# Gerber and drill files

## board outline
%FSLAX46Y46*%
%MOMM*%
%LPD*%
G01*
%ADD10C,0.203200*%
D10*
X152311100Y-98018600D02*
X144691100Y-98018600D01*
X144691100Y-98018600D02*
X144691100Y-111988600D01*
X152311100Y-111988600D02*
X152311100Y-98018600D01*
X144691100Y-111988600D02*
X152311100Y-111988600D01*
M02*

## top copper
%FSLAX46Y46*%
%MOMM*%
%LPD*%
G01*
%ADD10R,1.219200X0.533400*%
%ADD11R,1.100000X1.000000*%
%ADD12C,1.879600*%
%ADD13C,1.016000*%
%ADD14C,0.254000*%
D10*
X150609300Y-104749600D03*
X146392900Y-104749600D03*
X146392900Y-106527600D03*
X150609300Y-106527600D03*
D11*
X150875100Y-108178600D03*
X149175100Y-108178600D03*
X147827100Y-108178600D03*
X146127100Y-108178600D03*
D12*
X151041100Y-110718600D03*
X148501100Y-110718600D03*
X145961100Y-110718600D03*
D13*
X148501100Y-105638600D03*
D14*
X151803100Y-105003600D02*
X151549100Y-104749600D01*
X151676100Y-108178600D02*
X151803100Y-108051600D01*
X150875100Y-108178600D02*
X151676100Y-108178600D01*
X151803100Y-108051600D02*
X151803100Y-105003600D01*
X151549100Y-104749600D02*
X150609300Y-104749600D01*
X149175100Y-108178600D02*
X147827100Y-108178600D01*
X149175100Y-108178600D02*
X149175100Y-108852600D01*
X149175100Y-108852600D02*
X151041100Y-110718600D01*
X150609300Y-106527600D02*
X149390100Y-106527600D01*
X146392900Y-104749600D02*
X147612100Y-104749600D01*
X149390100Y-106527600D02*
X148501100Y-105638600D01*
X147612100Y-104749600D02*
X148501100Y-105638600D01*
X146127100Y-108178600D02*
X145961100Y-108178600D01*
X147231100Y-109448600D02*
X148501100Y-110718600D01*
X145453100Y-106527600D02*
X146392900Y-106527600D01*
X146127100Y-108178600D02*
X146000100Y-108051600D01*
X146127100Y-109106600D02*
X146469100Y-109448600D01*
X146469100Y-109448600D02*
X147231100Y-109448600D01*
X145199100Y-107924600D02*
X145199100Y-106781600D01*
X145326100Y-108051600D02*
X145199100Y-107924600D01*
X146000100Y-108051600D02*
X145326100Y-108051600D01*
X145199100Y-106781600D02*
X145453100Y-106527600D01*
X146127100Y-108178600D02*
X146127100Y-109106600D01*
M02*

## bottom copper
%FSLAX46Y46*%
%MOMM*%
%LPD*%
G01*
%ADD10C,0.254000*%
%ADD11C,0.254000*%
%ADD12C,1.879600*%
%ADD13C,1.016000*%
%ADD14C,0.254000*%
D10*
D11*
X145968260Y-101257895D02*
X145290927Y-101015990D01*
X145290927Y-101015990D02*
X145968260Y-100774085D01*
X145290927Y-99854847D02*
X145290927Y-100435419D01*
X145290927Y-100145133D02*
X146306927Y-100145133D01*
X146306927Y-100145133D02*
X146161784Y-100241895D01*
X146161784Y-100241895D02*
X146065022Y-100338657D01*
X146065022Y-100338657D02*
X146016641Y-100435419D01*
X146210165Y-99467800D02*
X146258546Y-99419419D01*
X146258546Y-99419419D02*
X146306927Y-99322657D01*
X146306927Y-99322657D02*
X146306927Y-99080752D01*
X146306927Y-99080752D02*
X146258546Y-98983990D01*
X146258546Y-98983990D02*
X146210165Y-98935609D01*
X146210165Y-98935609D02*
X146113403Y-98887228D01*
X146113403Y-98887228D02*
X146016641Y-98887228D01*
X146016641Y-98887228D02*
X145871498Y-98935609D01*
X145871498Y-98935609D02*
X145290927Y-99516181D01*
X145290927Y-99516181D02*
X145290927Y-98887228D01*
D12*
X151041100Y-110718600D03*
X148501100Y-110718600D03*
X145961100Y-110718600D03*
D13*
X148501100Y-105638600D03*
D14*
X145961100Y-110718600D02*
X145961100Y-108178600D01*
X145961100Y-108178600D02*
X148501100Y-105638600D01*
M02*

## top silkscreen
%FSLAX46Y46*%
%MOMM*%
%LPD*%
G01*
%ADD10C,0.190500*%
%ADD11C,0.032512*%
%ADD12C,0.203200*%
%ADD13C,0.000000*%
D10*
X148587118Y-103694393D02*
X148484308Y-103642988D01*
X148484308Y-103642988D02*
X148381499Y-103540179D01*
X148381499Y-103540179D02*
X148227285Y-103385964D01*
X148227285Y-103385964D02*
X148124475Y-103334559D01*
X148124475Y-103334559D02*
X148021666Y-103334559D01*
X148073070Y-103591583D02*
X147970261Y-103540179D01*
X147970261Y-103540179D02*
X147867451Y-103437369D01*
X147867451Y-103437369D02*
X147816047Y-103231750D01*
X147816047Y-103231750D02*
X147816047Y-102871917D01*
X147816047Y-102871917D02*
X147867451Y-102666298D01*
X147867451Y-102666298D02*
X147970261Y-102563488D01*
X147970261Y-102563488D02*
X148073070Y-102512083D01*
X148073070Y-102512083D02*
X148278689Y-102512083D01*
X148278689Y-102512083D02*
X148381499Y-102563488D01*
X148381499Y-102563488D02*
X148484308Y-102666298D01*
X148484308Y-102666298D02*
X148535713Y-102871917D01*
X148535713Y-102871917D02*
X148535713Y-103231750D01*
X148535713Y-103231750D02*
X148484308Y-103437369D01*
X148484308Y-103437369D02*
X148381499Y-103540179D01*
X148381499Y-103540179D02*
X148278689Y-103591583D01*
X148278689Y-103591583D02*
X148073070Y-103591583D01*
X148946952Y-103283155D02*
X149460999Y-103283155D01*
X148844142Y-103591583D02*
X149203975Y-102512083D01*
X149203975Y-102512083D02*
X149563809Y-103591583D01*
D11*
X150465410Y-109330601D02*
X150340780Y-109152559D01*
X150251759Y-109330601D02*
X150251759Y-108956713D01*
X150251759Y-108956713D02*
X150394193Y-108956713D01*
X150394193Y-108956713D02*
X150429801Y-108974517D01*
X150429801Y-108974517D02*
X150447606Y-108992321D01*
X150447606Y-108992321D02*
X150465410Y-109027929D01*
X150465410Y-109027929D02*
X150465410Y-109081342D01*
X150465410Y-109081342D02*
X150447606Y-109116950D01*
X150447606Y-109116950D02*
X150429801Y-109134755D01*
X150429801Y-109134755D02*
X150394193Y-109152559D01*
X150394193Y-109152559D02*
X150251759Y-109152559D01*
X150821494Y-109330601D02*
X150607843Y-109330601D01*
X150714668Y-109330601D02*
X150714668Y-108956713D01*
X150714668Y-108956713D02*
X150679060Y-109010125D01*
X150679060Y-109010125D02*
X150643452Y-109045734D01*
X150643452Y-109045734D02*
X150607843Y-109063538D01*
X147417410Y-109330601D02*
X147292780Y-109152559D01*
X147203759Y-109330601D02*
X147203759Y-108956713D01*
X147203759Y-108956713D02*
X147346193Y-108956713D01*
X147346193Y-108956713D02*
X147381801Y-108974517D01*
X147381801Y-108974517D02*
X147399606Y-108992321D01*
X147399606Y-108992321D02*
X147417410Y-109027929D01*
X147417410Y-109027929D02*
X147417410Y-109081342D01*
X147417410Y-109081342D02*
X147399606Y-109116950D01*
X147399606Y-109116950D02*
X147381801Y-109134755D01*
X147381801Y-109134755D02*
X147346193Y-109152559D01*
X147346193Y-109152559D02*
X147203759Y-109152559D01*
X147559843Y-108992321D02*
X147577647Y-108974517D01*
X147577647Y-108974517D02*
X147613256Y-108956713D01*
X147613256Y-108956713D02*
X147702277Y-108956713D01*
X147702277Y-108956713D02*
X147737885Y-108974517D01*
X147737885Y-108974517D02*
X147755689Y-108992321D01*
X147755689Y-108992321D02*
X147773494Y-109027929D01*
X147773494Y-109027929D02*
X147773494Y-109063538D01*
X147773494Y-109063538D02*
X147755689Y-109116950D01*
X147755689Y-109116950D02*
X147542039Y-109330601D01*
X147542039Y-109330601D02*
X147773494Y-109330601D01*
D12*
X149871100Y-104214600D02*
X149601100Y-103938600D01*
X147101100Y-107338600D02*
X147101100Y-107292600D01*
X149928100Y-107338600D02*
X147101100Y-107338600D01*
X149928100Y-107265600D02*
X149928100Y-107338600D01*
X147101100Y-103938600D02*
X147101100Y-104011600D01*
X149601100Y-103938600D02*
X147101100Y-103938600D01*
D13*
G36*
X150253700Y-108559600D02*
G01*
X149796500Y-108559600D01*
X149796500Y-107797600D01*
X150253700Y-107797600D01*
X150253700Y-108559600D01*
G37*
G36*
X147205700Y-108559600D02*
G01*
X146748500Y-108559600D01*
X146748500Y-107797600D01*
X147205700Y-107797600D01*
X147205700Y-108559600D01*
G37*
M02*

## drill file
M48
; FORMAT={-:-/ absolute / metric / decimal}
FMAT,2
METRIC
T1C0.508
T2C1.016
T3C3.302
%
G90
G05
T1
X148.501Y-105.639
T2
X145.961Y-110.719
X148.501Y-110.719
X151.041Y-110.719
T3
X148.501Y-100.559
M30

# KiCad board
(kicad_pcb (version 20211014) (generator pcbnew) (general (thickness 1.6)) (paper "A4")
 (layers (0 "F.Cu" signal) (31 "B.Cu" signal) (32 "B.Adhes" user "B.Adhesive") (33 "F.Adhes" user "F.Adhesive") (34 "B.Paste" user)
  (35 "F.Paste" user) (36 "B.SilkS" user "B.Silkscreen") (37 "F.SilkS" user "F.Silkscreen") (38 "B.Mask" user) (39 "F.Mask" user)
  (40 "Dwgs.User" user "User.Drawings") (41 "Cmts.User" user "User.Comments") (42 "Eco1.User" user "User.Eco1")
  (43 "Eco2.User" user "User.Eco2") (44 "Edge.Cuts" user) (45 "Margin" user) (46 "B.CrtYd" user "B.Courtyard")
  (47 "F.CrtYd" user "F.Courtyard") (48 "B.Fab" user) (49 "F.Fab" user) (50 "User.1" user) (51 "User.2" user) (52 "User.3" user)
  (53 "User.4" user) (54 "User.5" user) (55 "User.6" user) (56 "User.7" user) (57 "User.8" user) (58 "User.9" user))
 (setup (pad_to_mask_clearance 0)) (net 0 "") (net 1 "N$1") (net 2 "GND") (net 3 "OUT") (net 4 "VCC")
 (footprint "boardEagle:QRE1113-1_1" (layer "F.Cu") (at 148.5011 105.6386 180)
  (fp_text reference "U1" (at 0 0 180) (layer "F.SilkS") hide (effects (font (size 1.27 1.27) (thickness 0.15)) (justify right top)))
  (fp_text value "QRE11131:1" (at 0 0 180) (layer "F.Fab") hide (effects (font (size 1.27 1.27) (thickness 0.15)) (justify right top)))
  (fp_line (start -1.37 1.424) (end -1.1 1.7) (layer "F.SilkS") (width 0.2032))
  (fp_line (start 1.4 -1.7) (end 1.4 -1.654) (layer "F.SilkS") (width 0.2032))
  (fp_line (start -1.427 -1.7) (end 1.4 -1.7) (layer "F.SilkS") (width 0.2032))
  (fp_line (start -1.427 -1.627) (end -1.427 -1.7) (layer "F.SilkS") (width 0.2032))
  (fp_line (start 1.4 1.7) (end 1.4 1.627) (layer "F.SilkS") (width 0.2032))
  (fp_line (start -1.1 1.7) (end 1.4 1.7) (layer "F.SilkS") (width 0.2032))
  (pad "1" smd rect (at -2.1082 0.889 180) (size 1.2192 0.5334) (layers "F.Cu" "F.Paste" "F.Mask") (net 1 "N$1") (solder_mask_margin 0.1016))
  (pad "2" smd rect (at 2.1082 0.889 180) (size 1.2192 0.5334) (layers "F.Cu" "F.Paste" "F.Mask") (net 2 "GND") (solder_mask_margin 0.1016))
  (pad "3" smd rect (at 2.1082 -0.889 180) (size 1.2192 0.5334) (layers "F.Cu" "F.Paste" "F.Mask") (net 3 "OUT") (solder_mask_margin 0.1016))
  (pad "4" smd rect (at -2.1082 -0.889 180) (size 1.2192 0.5334) (layers "F.Cu" "F.Paste" "F.Mask") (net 2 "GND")
   (solder_mask_margin 0.1016)))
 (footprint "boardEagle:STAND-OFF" (layer "F.Cu") (at 148.5011 100.5586)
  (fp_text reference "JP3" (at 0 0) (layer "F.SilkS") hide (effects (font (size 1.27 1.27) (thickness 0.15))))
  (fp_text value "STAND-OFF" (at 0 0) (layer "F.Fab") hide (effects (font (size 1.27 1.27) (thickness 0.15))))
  (pad "" np_thru_hole circle (at 0 0) (size 3.302 3.302) (drill 3.302) (layers *.Cu *.Mask)))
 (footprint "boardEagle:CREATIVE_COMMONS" (layer "F.Cu") (at 166.2811 119.6086)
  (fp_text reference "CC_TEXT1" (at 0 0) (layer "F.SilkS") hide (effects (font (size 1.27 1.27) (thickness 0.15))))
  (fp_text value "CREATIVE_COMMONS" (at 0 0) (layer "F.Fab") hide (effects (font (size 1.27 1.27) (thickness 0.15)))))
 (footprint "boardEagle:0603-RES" (layer "F.Cu") (at 150.0251 108.1786 180)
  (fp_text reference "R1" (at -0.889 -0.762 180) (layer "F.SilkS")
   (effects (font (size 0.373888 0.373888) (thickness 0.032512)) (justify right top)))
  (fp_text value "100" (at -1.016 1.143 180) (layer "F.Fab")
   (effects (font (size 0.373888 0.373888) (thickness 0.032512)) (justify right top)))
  (fp_poly (pts (xy -0.2286 0.381) (xy 0.2286 0.381) (xy 0.2286 -0.381) (xy -0.2286 -0.381)) (layer "F.SilkS") (width 0) (fill solid))
  (pad "1" smd rect (at -0.85 0 180) (size 1.1 1) (layers "F.Cu" "F.Paste" "F.Mask") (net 1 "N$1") (solder_mask_margin 0.1016))
  (pad "2" smd rect (at 0.85 0 180) (size 1.1 1) (layers "F.Cu" "F.Paste" "F.Mask") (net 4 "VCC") (solder_mask_margin 0.1016)))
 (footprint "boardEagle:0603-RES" (layer "F.Cu") (at 146.9771 108.1786 180)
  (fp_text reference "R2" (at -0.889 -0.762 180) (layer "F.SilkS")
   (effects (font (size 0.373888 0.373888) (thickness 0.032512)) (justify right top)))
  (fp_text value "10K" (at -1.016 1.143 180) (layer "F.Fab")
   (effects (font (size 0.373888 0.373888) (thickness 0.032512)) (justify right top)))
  (fp_poly (pts (xy -0.2286 0.381) (xy 0.2286 0.381) (xy 0.2286 -0.381) (xy -0.2286 -0.381)) (layer "F.SilkS") (width 0) (fill solid))
  (pad "1" smd rect (at -0.85 0 180) (size 1.1 1) (layers "F.Cu" "F.Paste" "F.Mask") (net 4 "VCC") (solder_mask_margin 0.1016))
  (pad "2" smd rect (at 0.85 0 180) (size 1.1 1) (layers "F.Cu" "F.Paste" "F.Mask") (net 3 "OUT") (solder_mask_margin 0.1016)))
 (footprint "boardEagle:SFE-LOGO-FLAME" (layer "B.Cu") (at 151.1681 105.1306 180)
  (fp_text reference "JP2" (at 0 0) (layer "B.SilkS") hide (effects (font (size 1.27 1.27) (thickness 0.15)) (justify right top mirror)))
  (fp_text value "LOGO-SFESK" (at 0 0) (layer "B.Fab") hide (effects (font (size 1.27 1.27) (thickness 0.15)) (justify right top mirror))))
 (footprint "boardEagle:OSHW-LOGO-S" (layer "B.Cu") (at 146.7231 103.8606 180)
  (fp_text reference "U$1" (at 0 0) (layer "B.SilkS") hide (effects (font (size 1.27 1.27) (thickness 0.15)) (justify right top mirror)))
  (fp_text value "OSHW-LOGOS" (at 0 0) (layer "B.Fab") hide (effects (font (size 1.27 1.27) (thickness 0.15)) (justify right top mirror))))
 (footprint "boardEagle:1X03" (layer "B.Cu") (at 151.0411 110.7186 180)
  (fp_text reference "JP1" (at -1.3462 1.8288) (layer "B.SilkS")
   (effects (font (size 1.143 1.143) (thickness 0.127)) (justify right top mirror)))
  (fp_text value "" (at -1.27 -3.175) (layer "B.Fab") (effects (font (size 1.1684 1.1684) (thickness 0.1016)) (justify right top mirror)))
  (pad "1" thru_hole circle (at 0 0 90) (size 1.8796 1.8796) (drill 1.016) (layers *.Cu *.Mask) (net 4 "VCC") (solder_mask_margin 0.1016))
  (pad "2" thru_hole circle (at 2.54 0 90) (size 1.8796 1.8796) (drill 1.016) (layers *.Cu *.Mask) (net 3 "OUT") (solder_mask_margin 0.1016))
  (pad "3" thru_hole circle (at 5.08 0 90) (size 1.8796 1.8796) (drill 1.016) (layers *.Cu *.Mask) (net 2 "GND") (solder_mask_margin 0.1016)))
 (gr_line (start 152.3111 98.0186) (end 144.6911 98.0186) (layer "Edge.Cuts") (width 0.2032))
 (gr_line (start 144.6911 98.0186) (end 144.6911 111.9886) (layer "Edge.Cuts") (width 0.2032))
 (gr_line (start 152.3111 111.9886) (end 152.3111 98.0186) (layer "Edge.Cuts") (width 0.2032))
 (gr_line (start 144.6911 111.9886) (end 152.3111 111.9886) (layer "Edge.Cuts") (width 0.2032))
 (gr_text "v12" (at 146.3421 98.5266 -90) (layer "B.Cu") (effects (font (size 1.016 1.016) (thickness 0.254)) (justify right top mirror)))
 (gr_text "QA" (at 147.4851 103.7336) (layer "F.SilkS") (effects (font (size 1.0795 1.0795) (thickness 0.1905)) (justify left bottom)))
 (segment (start 151.8031 105.0036) (end 151.5491 104.7496) (width 0.254) (layer "F.Cu") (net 1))
 (segment (start 151.6761 108.1786) (end 151.8031 108.0516) (width 0.254) (layer "F.Cu") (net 1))
 (segment (start 150.8751 108.1786) (end 151.6761 108.1786) (width 0.254) (layer "F.Cu") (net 1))
 (segment (start 151.8031 108.0516) (end 151.8031 105.0036) (width 0.254) (layer "F.Cu") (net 1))
 (segment (start 151.5491 104.7496) (end 150.6093 104.7496) (width 0.254) (layer "F.Cu") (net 1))
 (segment (start 149.1751 108.1786) (end 147.8271 108.1786) (width 0.254) (layer "F.Cu") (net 4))
 (segment (start 149.1751 108.1786) (end 149.1751 108.8526) (width 0.254) (layer "F.Cu") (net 4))
 (segment (start 149.1751 108.8526) (end 151.0411 110.7186) (width 0.254) (layer "F.Cu") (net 4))
 (segment (start 150.6093 106.5276) (end 149.3901 106.5276) (width 0.254) (layer "F.Cu") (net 2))
 (segment (start 146.3929 104.7496) (end 147.6121 104.7496) (width 0.254) (layer "F.Cu") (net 2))
 (segment (start 149.3901 106.5276) (end 148.5011 105.6386) (width 0.254) (layer "F.Cu") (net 2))
 (segment (start 147.6121 104.7496) (end 148.5011 105.6386) (width 0.254) (layer "F.Cu") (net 2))
 (via (at 148.5011 105.6386) (size 1.016) (drill 0.508) (layers "F.Cu" "B.Cu") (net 2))
 (segment (start 145.9611 110.7186) (end 145.9611 108.1786) (width 0.254) (layer "B.Cu") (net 2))
 (segment (start 145.9611 108.1786) (end 148.5011 105.6386) (width 0.254) (layer "B.Cu") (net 2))
 (segment (start 146.1271 108.1786) (end 145.9611 108.1786) (width 0.254) (layer "F.Cu") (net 3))
 (segment (start 147.2311 109.4486) (end 148.5011 110.7186) (width 0.254) (layer "F.Cu") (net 3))
 (segment (start 145.4531 106.5276) (end 146.3929 106.5276) (width 0.254) (layer "F.Cu") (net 3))
 (segment (start 146.1271 108.1786) (end 146.0001 108.0516) (width 0.254) (layer "F.Cu") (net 3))
 (segment (start 146.1271 109.1066) (end 146.4691 109.4486) (width 0.254) (layer "F.Cu") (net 3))
 (segment (start 146.4691 109.4486) (end 147.2311 109.4486) (width 0.254) (layer "F.Cu") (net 3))
 (segment (start 145.1991 107.9246) (end 145.1991 106.7816) (width 0.254) (layer "F.Cu") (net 3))
 (segment (start 145.3261 108.0516) (end 145.1991 107.9246) (width 0.254) (layer "F.Cu") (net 3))
 (segment (start 146.0001 108.0516) (end 145.3261 108.0516) (width 0.254) (layer "F.Cu") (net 3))
 (segment (start 145.1991 106.7816) (end 145.4531 106.5276) (width 0.254) (layer "F.Cu") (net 3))
 (segment (start 146.1271 108.1786) (end 146.1271 109.1066) (width 0.254) (layer "F.Cu") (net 3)))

